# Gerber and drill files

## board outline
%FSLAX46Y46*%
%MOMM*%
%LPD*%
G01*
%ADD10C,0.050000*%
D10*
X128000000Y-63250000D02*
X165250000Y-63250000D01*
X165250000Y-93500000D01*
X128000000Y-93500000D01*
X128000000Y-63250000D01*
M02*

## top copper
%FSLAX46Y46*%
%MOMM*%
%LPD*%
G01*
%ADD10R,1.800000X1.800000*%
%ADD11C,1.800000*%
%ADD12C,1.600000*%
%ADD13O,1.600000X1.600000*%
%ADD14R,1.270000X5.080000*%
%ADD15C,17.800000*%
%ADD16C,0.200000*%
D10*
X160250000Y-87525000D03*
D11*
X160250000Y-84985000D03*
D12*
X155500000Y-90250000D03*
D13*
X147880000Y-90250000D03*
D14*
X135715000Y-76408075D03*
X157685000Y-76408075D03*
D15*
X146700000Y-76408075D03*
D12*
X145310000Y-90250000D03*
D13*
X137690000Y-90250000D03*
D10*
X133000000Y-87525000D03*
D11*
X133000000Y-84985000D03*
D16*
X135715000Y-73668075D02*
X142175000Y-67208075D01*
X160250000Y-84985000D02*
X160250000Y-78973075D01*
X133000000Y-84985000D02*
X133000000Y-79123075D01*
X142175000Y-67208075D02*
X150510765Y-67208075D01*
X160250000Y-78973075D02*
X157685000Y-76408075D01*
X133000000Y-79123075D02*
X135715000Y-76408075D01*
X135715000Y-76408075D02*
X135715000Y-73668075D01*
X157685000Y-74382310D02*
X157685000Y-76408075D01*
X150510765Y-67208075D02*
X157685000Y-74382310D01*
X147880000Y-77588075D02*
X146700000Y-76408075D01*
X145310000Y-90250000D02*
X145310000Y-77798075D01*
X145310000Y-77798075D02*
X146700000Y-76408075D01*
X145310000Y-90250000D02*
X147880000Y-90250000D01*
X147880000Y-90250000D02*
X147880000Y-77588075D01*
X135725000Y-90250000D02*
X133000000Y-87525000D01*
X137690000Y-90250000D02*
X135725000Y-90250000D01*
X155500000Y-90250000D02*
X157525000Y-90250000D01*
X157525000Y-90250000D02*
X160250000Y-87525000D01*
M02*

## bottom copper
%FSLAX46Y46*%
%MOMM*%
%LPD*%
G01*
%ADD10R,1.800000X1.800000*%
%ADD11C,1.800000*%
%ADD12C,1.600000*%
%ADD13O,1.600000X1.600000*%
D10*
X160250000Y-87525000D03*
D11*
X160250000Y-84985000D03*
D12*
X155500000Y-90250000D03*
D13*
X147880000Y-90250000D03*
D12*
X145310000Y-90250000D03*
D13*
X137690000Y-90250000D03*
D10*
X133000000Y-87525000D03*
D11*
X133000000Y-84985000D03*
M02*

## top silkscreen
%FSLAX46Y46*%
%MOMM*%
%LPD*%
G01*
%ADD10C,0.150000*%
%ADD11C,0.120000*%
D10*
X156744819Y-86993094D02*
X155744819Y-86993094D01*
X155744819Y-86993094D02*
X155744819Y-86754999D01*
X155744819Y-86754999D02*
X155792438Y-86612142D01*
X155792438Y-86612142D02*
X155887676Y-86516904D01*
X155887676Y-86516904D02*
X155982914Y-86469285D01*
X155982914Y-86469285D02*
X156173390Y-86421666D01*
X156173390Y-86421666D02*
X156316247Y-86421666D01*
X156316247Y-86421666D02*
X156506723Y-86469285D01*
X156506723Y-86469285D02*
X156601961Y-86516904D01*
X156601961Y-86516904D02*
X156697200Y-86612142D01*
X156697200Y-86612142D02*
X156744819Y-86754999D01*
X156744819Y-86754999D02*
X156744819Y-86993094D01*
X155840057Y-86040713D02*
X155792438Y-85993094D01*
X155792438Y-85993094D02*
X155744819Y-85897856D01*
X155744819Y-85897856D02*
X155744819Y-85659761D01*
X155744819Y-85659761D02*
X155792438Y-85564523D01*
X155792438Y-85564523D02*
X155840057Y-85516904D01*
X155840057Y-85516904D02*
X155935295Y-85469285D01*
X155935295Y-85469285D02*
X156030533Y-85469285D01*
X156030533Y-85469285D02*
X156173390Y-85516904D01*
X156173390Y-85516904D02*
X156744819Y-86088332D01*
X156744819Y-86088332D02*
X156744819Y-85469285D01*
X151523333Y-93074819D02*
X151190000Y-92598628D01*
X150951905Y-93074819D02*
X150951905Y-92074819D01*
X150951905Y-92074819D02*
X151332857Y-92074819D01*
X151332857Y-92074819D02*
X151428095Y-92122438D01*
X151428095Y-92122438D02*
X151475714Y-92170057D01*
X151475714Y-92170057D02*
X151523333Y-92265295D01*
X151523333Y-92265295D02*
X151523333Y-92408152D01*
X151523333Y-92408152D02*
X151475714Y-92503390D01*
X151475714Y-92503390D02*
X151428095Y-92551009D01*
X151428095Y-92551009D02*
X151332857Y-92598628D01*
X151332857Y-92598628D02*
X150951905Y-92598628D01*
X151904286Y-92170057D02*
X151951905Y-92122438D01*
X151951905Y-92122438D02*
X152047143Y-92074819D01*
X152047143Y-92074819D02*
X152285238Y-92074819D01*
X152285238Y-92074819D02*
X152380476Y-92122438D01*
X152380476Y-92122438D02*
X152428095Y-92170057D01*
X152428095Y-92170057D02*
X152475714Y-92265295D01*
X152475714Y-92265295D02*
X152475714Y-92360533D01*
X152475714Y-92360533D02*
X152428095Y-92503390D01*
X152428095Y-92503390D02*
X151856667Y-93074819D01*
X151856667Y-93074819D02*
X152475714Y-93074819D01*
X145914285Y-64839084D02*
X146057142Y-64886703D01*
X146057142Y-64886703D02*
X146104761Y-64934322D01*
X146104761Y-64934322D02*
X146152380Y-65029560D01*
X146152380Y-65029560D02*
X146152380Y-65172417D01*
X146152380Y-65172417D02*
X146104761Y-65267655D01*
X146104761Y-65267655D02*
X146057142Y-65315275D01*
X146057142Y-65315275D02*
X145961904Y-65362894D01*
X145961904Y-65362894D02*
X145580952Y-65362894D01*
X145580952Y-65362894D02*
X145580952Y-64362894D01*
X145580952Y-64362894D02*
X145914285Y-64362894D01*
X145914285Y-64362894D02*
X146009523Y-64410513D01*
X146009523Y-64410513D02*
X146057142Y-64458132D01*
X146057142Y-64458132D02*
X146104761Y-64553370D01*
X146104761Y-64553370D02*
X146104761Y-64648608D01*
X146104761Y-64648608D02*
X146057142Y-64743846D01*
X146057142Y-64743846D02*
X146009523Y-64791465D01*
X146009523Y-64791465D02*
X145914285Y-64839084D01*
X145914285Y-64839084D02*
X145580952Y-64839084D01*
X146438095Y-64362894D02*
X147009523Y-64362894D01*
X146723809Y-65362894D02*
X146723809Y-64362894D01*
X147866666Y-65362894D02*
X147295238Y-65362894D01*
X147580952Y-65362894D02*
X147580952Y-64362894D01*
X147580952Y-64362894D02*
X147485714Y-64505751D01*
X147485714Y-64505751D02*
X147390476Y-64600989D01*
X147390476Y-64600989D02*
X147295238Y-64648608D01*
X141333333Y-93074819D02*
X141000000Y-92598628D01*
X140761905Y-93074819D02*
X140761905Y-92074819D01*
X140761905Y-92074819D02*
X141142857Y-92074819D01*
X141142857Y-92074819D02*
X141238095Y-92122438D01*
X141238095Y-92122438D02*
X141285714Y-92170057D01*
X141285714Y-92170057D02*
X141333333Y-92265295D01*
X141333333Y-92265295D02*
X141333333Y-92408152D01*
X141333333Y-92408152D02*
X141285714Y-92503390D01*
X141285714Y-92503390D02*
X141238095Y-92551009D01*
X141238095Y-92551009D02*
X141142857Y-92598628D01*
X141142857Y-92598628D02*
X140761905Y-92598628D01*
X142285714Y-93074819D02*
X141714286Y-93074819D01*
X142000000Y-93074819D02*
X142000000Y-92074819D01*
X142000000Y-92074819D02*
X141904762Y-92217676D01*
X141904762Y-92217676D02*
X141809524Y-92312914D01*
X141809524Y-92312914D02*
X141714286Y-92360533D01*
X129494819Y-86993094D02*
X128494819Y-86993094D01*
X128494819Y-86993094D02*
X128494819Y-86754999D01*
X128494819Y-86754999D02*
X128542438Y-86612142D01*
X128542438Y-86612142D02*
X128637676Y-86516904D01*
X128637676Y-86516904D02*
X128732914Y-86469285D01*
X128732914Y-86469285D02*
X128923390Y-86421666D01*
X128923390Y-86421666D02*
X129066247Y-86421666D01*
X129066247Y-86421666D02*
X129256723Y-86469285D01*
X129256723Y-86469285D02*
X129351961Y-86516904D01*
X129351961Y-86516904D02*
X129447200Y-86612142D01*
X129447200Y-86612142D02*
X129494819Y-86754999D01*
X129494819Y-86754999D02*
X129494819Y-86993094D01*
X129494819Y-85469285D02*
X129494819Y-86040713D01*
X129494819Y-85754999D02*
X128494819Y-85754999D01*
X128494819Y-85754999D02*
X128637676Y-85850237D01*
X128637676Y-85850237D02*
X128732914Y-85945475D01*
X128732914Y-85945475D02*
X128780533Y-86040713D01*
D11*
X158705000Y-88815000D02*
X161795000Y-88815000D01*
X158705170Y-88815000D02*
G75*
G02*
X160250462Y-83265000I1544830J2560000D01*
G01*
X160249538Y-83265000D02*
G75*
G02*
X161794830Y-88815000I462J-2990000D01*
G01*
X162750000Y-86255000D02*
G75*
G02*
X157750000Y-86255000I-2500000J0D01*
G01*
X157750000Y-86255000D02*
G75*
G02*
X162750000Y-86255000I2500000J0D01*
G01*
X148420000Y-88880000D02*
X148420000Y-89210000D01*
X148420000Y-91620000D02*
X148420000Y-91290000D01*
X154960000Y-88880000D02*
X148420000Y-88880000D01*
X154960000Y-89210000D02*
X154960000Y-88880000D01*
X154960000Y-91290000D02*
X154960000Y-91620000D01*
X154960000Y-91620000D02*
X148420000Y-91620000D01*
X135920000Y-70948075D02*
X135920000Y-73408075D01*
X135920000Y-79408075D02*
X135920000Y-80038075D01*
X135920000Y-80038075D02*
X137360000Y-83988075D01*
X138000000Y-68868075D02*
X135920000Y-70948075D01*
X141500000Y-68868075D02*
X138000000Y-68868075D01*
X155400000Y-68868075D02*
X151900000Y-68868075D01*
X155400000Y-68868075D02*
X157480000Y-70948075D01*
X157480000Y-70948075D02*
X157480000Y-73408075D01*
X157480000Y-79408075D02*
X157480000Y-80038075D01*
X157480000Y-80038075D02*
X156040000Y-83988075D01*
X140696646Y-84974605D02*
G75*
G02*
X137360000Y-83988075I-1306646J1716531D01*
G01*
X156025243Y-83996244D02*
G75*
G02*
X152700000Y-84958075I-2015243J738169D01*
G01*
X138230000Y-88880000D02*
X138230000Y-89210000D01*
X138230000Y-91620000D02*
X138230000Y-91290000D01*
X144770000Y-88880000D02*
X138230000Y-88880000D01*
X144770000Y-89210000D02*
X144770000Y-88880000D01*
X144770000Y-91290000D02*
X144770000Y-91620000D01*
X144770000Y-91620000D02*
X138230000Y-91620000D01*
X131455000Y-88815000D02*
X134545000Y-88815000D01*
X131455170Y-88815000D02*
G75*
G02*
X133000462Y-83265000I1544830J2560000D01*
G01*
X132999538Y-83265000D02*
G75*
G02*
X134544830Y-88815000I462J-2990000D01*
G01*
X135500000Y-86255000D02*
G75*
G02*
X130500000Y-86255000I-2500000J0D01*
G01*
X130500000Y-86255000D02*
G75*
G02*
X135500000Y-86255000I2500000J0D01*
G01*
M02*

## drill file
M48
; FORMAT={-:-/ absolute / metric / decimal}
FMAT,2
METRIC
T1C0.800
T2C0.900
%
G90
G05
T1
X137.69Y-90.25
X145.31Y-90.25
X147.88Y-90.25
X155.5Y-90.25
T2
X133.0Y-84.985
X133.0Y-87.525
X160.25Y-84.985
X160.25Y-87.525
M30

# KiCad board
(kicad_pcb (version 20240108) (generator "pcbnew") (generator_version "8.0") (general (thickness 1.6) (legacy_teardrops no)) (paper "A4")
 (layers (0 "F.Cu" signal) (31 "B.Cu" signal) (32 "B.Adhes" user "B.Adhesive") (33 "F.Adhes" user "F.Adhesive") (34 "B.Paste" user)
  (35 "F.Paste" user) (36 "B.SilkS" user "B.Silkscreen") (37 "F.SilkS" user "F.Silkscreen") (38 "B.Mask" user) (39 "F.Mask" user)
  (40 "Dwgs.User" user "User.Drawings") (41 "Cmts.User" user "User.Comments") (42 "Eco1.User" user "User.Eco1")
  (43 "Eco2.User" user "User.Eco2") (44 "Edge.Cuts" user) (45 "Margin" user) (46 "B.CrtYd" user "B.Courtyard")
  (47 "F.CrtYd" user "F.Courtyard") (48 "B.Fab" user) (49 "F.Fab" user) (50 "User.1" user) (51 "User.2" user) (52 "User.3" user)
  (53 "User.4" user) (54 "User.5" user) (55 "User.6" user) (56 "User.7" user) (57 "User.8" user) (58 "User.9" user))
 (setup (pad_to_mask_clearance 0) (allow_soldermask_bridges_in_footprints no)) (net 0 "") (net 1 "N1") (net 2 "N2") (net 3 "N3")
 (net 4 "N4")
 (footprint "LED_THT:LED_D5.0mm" (layer "F.Cu") (at 160.25 87.525 90)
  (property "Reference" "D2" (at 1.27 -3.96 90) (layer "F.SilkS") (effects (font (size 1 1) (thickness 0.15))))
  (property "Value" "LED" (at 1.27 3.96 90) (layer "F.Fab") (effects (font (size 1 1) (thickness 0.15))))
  (fp_line (start -1.29 -1.545) (end -1.29 1.545) (stroke (width 0.12) (type solid)) (layer "F.SilkS"))
  (fp_arc (start -1.29 -1.54483) (mid 2.072002 -2.880433) (end 4.26 0.000462) (stroke (width 0.12) (type solid)) (layer "F.SilkS"))
  (fp_arc (start 4.26 -0.000462) (mid 2.072002 2.880433) (end -1.29 1.54483) (stroke (width 0.12) (type solid)) (layer "F.SilkS"))
  (fp_circle (center 1.27 0) (end 3.77 0) (stroke (width 0.12) (type solid)) (fill none) (layer "F.SilkS"))
  (pad "1" thru_hole rect (at 0 0 90) (size 1.8 1.8) (drill 0.9) (layers "*.Cu" "*.Mask") (remove_unused_layers no) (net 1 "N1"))
  (pad "2" thru_hole circle (at 2.54 0 90) (size 1.8 1.8) (drill 0.9) (layers "*.Cu" "*.Mask") (remove_unused_layers no) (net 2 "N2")))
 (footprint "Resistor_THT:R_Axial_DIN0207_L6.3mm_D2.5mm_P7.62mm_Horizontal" (layer "F.Cu") (at 155.5 90.25 180)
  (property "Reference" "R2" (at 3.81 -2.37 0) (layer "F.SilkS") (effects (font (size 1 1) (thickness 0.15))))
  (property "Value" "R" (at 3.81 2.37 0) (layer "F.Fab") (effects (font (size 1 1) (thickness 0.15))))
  (fp_line (start 7.08 1.37) (end 7.08 1.04) (stroke (width 0.12) (type solid)) (layer "F.SilkS"))
  (fp_line (start 7.08 -1.37) (end 7.08 -1.04) (stroke (width 0.12) (type solid)) (layer "F.SilkS"))
  (fp_line (start 0.54 1.37) (end 7.08 1.37) (stroke (width 0.12) (type solid)) (layer "F.SilkS"))
  (fp_line (start 0.54 1.04) (end 0.54 1.37) (stroke (width 0.12) (type solid)) (layer "F.SilkS"))
  (fp_line (start 0.54 -1.04) (end 0.54 -1.37) (stroke (width 0.12) (type solid)) (layer "F.SilkS"))
  (fp_line (start 0.54 -1.37) (end 7.08 -1.37) (stroke (width 0.12) (type solid)) (layer "F.SilkS"))
  (pad "1" thru_hole circle (at 0 0 180) (size 1.6 1.6) (drill 0.8) (layers "*.Cu" "*.Mask") (remove_unused_layers no) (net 1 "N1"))
  (pad "2" thru_hole oval (at 7.62 0 180) (size 1.6 1.6) (drill 0.8) (layers "*.Cu" "*.Mask") (remove_unused_layers no) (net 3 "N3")))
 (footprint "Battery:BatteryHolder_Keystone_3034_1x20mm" (layer "F.Cu") (at 146.7 76.408075)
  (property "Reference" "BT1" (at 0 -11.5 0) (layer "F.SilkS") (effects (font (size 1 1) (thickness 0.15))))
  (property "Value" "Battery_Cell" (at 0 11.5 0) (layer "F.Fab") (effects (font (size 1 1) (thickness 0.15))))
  (fp_line (start -10.78 -5.46) (end -10.78 -3) (stroke (width 0.12) (type solid)) (layer "F.SilkS"))
  (fp_line (start -10.78 3) (end -10.78 3.63) (stroke (width 0.12) (type solid)) (layer "F.SilkS"))
  (fp_line (start -10.78 3.63) (end -9.34 7.58) (stroke (width 0.12) (type solid)) (layer "F.SilkS"))
  (fp_line (start -8.7 -7.54) (end -10.78 -5.46) (stroke (width 0.12) (type solid)) (layer "F.SilkS"))
  (fp_line (start -5.2 -7.54) (end -8.7 -7.54) (stroke (width 0.12) (type solid)) (layer "F.SilkS"))
  (fp_line (start 8.7 -7.54) (end 5.2 -7.54) (stroke (width 0.12) (type solid)) (layer "F.SilkS"))
  (fp_line (start 8.7 -7.54) (end 10.78 -5.46) (stroke (width 0.12) (type solid)) (layer "F.SilkS"))
  (fp_line (start 10.78 -5.46) (end 10.78 -3) (stroke (width 0.12) (type solid)) (layer "F.SilkS"))
  (fp_line (start 10.78 3) (end 10.78 3.63) (stroke (width 0.12) (type solid)) (layer "F.SilkS"))
  (fp_line (start 10.78 3.63) (end 9.34 7.58) (stroke (width 0.12) (type solid)) (layer "F.SilkS"))
  (fp_arc (start -6.003354 8.56653) (mid -7.921654 8.918738) (end -9.34 7.58) (stroke (width 0.12) (type solid)) (layer "F.SilkS"))
  (fp_arc (start 9.325243 7.588169) (mid 7.90634 8.911668) (end 6 8.55) (stroke (width 0.12) (type solid)) (layer "F.SilkS"))
  (pad "1" smd rect (at -10.985 0) (size 1.27 5.08) (layers "F.Cu" "F.Paste" "F.Mask") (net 2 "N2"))
  (pad "1" smd rect (at 10.985 0) (size 1.27 5.08) (layers "F.Cu" "F.Paste" "F.Mask") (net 2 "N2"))
  (pad "2" smd circle (at 0 0) (size 17.8 17.8) (layers "F.Cu" "F.Mask") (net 3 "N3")))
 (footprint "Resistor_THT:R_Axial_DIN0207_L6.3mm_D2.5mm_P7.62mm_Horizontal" (layer "F.Cu") (at 145.31 90.25 180)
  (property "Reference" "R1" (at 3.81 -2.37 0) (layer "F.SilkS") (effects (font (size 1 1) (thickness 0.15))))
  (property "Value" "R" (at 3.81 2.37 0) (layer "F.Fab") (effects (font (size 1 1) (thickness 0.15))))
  (fp_line (start 7.08 1.37) (end 7.08 1.04) (stroke (width 0.12) (type solid)) (layer "F.SilkS"))
  (fp_line (start 7.08 -1.37) (end 7.08 -1.04) (stroke (width 0.12) (type solid)) (layer "F.SilkS"))
  (fp_line (start 0.54 1.37) (end 7.08 1.37) (stroke (width 0.12) (type solid)) (layer "F.SilkS"))
  (fp_line (start 0.54 1.04) (end 0.54 1.37) (stroke (width 0.12) (type solid)) (layer "F.SilkS"))
  (fp_line (start 0.54 -1.04) (end 0.54 -1.37) (stroke (width 0.12) (type solid)) (layer "F.SilkS"))
  (fp_line (start 0.54 -1.37) (end 7.08 -1.37) (stroke (width 0.12) (type solid)) (layer "F.SilkS"))
  (pad "1" thru_hole circle (at 0 0 180) (size 1.6 1.6) (drill 0.8) (layers "*.Cu" "*.Mask") (remove_unused_layers no) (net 3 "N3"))
  (pad "2" thru_hole oval (at 7.62 0 180) (size 1.6 1.6) (drill 0.8) (layers "*.Cu" "*.Mask") (remove_unused_layers no) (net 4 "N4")))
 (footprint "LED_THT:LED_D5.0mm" (layer "F.Cu") (at 133 87.525 90)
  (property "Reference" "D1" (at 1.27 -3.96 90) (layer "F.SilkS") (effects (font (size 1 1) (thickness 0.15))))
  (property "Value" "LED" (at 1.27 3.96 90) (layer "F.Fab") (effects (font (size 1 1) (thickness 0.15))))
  (fp_line (start -1.29 -1.545) (end -1.29 1.545) (stroke (width 0.12) (type solid)) (layer "F.SilkS"))
  (fp_arc (start -1.29 -1.54483) (mid 2.072002 -2.880433) (end 4.26 0.000462) (stroke (width 0.12) (type solid)) (layer "F.SilkS"))
  (fp_arc (start 4.26 -0.000462) (mid 2.072002 2.880433) (end -1.29 1.54483) (stroke (width 0.12) (type solid)) (layer "F.SilkS"))
  (fp_circle (center 1.27 0) (end 3.77 0) (stroke (width 0.12) (type solid)) (fill none) (layer "F.SilkS"))
  (pad "1" thru_hole rect (at 0 0 90) (size 1.8 1.8) (drill 0.9) (layers "*.Cu" "*.Mask") (remove_unused_layers no) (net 4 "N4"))
  (pad "2" thru_hole circle (at 2.54 0 90) (size 1.8 1.8) (drill 0.9) (layers "*.Cu" "*.Mask") (remove_unused_layers no) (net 2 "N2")))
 (gr_rect (start 128 63.25) (end 165.25 93.5) (stroke (width 0.05) (type default)) (fill none) (layer "Edge.Cuts"))
 (segment (start 135.715 73.668075) (end 142.175 67.208075) (width 0.2) (layer "F.Cu") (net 2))
 (segment (start 160.25 84.985) (end 160.25 78.973075) (width 0.2) (layer "F.Cu") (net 2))
 (segment (start 133 84.985) (end 133 79.123075) (width 0.2) (layer "F.Cu") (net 2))
 (segment (start 142.175 67.208075) (end 150.510765 67.208075) (width 0.2) (layer "F.Cu") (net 2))
 (segment (start 160.25 78.973075) (end 157.685 76.408075) (width 0.2) (layer "F.Cu") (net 2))
 (segment (start 133 79.123075) (end 135.715 76.408075) (width 0.2) (layer "F.Cu") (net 2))
 (segment (start 135.715 76.408075) (end 135.715 73.668075) (width 0.2) (layer "F.Cu") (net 2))
 (segment (start 157.685 74.38231) (end 157.685 76.408075) (width 0.2) (layer "F.Cu") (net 2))
 (segment (start 150.510765 67.208075) (end 157.685 74.38231) (width 0.2) (layer "F.Cu") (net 2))
 (segment (start 147.88 77.588075) (end 146.7 76.408075) (width 0.2) (layer "F.Cu") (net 3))
 (segment (start 145.31 90.25) (end 145.31 77.798075) (width 0.2) (layer "F.Cu") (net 3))
 (segment (start 145.31 77.798075) (end 146.7 76.408075) (width 0.2) (layer "F.Cu") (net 3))
 (segment (start 145.31 90.25) (end 147.88 90.25) (width 0.2) (layer "F.Cu") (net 3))
 (segment (start 147.88 90.25) (end 147.88 77.588075) (width 0.2) (layer "F.Cu") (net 3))
 (segment (start 135.725 90.25) (end 133 87.525) (width 0.2) (layer "F.Cu") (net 4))
 (segment (start 137.69 90.25) (end 135.725 90.25) (width 0.2) (layer "F.Cu") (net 4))
 (segment (start 155.5 90.25) (end 157.525 90.25) (width 0.2) (layer "F.Cu") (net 1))
 (segment (start 157.525 90.25) (end 160.25 87.525) (width 0.2) (layer "F.Cu") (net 1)))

